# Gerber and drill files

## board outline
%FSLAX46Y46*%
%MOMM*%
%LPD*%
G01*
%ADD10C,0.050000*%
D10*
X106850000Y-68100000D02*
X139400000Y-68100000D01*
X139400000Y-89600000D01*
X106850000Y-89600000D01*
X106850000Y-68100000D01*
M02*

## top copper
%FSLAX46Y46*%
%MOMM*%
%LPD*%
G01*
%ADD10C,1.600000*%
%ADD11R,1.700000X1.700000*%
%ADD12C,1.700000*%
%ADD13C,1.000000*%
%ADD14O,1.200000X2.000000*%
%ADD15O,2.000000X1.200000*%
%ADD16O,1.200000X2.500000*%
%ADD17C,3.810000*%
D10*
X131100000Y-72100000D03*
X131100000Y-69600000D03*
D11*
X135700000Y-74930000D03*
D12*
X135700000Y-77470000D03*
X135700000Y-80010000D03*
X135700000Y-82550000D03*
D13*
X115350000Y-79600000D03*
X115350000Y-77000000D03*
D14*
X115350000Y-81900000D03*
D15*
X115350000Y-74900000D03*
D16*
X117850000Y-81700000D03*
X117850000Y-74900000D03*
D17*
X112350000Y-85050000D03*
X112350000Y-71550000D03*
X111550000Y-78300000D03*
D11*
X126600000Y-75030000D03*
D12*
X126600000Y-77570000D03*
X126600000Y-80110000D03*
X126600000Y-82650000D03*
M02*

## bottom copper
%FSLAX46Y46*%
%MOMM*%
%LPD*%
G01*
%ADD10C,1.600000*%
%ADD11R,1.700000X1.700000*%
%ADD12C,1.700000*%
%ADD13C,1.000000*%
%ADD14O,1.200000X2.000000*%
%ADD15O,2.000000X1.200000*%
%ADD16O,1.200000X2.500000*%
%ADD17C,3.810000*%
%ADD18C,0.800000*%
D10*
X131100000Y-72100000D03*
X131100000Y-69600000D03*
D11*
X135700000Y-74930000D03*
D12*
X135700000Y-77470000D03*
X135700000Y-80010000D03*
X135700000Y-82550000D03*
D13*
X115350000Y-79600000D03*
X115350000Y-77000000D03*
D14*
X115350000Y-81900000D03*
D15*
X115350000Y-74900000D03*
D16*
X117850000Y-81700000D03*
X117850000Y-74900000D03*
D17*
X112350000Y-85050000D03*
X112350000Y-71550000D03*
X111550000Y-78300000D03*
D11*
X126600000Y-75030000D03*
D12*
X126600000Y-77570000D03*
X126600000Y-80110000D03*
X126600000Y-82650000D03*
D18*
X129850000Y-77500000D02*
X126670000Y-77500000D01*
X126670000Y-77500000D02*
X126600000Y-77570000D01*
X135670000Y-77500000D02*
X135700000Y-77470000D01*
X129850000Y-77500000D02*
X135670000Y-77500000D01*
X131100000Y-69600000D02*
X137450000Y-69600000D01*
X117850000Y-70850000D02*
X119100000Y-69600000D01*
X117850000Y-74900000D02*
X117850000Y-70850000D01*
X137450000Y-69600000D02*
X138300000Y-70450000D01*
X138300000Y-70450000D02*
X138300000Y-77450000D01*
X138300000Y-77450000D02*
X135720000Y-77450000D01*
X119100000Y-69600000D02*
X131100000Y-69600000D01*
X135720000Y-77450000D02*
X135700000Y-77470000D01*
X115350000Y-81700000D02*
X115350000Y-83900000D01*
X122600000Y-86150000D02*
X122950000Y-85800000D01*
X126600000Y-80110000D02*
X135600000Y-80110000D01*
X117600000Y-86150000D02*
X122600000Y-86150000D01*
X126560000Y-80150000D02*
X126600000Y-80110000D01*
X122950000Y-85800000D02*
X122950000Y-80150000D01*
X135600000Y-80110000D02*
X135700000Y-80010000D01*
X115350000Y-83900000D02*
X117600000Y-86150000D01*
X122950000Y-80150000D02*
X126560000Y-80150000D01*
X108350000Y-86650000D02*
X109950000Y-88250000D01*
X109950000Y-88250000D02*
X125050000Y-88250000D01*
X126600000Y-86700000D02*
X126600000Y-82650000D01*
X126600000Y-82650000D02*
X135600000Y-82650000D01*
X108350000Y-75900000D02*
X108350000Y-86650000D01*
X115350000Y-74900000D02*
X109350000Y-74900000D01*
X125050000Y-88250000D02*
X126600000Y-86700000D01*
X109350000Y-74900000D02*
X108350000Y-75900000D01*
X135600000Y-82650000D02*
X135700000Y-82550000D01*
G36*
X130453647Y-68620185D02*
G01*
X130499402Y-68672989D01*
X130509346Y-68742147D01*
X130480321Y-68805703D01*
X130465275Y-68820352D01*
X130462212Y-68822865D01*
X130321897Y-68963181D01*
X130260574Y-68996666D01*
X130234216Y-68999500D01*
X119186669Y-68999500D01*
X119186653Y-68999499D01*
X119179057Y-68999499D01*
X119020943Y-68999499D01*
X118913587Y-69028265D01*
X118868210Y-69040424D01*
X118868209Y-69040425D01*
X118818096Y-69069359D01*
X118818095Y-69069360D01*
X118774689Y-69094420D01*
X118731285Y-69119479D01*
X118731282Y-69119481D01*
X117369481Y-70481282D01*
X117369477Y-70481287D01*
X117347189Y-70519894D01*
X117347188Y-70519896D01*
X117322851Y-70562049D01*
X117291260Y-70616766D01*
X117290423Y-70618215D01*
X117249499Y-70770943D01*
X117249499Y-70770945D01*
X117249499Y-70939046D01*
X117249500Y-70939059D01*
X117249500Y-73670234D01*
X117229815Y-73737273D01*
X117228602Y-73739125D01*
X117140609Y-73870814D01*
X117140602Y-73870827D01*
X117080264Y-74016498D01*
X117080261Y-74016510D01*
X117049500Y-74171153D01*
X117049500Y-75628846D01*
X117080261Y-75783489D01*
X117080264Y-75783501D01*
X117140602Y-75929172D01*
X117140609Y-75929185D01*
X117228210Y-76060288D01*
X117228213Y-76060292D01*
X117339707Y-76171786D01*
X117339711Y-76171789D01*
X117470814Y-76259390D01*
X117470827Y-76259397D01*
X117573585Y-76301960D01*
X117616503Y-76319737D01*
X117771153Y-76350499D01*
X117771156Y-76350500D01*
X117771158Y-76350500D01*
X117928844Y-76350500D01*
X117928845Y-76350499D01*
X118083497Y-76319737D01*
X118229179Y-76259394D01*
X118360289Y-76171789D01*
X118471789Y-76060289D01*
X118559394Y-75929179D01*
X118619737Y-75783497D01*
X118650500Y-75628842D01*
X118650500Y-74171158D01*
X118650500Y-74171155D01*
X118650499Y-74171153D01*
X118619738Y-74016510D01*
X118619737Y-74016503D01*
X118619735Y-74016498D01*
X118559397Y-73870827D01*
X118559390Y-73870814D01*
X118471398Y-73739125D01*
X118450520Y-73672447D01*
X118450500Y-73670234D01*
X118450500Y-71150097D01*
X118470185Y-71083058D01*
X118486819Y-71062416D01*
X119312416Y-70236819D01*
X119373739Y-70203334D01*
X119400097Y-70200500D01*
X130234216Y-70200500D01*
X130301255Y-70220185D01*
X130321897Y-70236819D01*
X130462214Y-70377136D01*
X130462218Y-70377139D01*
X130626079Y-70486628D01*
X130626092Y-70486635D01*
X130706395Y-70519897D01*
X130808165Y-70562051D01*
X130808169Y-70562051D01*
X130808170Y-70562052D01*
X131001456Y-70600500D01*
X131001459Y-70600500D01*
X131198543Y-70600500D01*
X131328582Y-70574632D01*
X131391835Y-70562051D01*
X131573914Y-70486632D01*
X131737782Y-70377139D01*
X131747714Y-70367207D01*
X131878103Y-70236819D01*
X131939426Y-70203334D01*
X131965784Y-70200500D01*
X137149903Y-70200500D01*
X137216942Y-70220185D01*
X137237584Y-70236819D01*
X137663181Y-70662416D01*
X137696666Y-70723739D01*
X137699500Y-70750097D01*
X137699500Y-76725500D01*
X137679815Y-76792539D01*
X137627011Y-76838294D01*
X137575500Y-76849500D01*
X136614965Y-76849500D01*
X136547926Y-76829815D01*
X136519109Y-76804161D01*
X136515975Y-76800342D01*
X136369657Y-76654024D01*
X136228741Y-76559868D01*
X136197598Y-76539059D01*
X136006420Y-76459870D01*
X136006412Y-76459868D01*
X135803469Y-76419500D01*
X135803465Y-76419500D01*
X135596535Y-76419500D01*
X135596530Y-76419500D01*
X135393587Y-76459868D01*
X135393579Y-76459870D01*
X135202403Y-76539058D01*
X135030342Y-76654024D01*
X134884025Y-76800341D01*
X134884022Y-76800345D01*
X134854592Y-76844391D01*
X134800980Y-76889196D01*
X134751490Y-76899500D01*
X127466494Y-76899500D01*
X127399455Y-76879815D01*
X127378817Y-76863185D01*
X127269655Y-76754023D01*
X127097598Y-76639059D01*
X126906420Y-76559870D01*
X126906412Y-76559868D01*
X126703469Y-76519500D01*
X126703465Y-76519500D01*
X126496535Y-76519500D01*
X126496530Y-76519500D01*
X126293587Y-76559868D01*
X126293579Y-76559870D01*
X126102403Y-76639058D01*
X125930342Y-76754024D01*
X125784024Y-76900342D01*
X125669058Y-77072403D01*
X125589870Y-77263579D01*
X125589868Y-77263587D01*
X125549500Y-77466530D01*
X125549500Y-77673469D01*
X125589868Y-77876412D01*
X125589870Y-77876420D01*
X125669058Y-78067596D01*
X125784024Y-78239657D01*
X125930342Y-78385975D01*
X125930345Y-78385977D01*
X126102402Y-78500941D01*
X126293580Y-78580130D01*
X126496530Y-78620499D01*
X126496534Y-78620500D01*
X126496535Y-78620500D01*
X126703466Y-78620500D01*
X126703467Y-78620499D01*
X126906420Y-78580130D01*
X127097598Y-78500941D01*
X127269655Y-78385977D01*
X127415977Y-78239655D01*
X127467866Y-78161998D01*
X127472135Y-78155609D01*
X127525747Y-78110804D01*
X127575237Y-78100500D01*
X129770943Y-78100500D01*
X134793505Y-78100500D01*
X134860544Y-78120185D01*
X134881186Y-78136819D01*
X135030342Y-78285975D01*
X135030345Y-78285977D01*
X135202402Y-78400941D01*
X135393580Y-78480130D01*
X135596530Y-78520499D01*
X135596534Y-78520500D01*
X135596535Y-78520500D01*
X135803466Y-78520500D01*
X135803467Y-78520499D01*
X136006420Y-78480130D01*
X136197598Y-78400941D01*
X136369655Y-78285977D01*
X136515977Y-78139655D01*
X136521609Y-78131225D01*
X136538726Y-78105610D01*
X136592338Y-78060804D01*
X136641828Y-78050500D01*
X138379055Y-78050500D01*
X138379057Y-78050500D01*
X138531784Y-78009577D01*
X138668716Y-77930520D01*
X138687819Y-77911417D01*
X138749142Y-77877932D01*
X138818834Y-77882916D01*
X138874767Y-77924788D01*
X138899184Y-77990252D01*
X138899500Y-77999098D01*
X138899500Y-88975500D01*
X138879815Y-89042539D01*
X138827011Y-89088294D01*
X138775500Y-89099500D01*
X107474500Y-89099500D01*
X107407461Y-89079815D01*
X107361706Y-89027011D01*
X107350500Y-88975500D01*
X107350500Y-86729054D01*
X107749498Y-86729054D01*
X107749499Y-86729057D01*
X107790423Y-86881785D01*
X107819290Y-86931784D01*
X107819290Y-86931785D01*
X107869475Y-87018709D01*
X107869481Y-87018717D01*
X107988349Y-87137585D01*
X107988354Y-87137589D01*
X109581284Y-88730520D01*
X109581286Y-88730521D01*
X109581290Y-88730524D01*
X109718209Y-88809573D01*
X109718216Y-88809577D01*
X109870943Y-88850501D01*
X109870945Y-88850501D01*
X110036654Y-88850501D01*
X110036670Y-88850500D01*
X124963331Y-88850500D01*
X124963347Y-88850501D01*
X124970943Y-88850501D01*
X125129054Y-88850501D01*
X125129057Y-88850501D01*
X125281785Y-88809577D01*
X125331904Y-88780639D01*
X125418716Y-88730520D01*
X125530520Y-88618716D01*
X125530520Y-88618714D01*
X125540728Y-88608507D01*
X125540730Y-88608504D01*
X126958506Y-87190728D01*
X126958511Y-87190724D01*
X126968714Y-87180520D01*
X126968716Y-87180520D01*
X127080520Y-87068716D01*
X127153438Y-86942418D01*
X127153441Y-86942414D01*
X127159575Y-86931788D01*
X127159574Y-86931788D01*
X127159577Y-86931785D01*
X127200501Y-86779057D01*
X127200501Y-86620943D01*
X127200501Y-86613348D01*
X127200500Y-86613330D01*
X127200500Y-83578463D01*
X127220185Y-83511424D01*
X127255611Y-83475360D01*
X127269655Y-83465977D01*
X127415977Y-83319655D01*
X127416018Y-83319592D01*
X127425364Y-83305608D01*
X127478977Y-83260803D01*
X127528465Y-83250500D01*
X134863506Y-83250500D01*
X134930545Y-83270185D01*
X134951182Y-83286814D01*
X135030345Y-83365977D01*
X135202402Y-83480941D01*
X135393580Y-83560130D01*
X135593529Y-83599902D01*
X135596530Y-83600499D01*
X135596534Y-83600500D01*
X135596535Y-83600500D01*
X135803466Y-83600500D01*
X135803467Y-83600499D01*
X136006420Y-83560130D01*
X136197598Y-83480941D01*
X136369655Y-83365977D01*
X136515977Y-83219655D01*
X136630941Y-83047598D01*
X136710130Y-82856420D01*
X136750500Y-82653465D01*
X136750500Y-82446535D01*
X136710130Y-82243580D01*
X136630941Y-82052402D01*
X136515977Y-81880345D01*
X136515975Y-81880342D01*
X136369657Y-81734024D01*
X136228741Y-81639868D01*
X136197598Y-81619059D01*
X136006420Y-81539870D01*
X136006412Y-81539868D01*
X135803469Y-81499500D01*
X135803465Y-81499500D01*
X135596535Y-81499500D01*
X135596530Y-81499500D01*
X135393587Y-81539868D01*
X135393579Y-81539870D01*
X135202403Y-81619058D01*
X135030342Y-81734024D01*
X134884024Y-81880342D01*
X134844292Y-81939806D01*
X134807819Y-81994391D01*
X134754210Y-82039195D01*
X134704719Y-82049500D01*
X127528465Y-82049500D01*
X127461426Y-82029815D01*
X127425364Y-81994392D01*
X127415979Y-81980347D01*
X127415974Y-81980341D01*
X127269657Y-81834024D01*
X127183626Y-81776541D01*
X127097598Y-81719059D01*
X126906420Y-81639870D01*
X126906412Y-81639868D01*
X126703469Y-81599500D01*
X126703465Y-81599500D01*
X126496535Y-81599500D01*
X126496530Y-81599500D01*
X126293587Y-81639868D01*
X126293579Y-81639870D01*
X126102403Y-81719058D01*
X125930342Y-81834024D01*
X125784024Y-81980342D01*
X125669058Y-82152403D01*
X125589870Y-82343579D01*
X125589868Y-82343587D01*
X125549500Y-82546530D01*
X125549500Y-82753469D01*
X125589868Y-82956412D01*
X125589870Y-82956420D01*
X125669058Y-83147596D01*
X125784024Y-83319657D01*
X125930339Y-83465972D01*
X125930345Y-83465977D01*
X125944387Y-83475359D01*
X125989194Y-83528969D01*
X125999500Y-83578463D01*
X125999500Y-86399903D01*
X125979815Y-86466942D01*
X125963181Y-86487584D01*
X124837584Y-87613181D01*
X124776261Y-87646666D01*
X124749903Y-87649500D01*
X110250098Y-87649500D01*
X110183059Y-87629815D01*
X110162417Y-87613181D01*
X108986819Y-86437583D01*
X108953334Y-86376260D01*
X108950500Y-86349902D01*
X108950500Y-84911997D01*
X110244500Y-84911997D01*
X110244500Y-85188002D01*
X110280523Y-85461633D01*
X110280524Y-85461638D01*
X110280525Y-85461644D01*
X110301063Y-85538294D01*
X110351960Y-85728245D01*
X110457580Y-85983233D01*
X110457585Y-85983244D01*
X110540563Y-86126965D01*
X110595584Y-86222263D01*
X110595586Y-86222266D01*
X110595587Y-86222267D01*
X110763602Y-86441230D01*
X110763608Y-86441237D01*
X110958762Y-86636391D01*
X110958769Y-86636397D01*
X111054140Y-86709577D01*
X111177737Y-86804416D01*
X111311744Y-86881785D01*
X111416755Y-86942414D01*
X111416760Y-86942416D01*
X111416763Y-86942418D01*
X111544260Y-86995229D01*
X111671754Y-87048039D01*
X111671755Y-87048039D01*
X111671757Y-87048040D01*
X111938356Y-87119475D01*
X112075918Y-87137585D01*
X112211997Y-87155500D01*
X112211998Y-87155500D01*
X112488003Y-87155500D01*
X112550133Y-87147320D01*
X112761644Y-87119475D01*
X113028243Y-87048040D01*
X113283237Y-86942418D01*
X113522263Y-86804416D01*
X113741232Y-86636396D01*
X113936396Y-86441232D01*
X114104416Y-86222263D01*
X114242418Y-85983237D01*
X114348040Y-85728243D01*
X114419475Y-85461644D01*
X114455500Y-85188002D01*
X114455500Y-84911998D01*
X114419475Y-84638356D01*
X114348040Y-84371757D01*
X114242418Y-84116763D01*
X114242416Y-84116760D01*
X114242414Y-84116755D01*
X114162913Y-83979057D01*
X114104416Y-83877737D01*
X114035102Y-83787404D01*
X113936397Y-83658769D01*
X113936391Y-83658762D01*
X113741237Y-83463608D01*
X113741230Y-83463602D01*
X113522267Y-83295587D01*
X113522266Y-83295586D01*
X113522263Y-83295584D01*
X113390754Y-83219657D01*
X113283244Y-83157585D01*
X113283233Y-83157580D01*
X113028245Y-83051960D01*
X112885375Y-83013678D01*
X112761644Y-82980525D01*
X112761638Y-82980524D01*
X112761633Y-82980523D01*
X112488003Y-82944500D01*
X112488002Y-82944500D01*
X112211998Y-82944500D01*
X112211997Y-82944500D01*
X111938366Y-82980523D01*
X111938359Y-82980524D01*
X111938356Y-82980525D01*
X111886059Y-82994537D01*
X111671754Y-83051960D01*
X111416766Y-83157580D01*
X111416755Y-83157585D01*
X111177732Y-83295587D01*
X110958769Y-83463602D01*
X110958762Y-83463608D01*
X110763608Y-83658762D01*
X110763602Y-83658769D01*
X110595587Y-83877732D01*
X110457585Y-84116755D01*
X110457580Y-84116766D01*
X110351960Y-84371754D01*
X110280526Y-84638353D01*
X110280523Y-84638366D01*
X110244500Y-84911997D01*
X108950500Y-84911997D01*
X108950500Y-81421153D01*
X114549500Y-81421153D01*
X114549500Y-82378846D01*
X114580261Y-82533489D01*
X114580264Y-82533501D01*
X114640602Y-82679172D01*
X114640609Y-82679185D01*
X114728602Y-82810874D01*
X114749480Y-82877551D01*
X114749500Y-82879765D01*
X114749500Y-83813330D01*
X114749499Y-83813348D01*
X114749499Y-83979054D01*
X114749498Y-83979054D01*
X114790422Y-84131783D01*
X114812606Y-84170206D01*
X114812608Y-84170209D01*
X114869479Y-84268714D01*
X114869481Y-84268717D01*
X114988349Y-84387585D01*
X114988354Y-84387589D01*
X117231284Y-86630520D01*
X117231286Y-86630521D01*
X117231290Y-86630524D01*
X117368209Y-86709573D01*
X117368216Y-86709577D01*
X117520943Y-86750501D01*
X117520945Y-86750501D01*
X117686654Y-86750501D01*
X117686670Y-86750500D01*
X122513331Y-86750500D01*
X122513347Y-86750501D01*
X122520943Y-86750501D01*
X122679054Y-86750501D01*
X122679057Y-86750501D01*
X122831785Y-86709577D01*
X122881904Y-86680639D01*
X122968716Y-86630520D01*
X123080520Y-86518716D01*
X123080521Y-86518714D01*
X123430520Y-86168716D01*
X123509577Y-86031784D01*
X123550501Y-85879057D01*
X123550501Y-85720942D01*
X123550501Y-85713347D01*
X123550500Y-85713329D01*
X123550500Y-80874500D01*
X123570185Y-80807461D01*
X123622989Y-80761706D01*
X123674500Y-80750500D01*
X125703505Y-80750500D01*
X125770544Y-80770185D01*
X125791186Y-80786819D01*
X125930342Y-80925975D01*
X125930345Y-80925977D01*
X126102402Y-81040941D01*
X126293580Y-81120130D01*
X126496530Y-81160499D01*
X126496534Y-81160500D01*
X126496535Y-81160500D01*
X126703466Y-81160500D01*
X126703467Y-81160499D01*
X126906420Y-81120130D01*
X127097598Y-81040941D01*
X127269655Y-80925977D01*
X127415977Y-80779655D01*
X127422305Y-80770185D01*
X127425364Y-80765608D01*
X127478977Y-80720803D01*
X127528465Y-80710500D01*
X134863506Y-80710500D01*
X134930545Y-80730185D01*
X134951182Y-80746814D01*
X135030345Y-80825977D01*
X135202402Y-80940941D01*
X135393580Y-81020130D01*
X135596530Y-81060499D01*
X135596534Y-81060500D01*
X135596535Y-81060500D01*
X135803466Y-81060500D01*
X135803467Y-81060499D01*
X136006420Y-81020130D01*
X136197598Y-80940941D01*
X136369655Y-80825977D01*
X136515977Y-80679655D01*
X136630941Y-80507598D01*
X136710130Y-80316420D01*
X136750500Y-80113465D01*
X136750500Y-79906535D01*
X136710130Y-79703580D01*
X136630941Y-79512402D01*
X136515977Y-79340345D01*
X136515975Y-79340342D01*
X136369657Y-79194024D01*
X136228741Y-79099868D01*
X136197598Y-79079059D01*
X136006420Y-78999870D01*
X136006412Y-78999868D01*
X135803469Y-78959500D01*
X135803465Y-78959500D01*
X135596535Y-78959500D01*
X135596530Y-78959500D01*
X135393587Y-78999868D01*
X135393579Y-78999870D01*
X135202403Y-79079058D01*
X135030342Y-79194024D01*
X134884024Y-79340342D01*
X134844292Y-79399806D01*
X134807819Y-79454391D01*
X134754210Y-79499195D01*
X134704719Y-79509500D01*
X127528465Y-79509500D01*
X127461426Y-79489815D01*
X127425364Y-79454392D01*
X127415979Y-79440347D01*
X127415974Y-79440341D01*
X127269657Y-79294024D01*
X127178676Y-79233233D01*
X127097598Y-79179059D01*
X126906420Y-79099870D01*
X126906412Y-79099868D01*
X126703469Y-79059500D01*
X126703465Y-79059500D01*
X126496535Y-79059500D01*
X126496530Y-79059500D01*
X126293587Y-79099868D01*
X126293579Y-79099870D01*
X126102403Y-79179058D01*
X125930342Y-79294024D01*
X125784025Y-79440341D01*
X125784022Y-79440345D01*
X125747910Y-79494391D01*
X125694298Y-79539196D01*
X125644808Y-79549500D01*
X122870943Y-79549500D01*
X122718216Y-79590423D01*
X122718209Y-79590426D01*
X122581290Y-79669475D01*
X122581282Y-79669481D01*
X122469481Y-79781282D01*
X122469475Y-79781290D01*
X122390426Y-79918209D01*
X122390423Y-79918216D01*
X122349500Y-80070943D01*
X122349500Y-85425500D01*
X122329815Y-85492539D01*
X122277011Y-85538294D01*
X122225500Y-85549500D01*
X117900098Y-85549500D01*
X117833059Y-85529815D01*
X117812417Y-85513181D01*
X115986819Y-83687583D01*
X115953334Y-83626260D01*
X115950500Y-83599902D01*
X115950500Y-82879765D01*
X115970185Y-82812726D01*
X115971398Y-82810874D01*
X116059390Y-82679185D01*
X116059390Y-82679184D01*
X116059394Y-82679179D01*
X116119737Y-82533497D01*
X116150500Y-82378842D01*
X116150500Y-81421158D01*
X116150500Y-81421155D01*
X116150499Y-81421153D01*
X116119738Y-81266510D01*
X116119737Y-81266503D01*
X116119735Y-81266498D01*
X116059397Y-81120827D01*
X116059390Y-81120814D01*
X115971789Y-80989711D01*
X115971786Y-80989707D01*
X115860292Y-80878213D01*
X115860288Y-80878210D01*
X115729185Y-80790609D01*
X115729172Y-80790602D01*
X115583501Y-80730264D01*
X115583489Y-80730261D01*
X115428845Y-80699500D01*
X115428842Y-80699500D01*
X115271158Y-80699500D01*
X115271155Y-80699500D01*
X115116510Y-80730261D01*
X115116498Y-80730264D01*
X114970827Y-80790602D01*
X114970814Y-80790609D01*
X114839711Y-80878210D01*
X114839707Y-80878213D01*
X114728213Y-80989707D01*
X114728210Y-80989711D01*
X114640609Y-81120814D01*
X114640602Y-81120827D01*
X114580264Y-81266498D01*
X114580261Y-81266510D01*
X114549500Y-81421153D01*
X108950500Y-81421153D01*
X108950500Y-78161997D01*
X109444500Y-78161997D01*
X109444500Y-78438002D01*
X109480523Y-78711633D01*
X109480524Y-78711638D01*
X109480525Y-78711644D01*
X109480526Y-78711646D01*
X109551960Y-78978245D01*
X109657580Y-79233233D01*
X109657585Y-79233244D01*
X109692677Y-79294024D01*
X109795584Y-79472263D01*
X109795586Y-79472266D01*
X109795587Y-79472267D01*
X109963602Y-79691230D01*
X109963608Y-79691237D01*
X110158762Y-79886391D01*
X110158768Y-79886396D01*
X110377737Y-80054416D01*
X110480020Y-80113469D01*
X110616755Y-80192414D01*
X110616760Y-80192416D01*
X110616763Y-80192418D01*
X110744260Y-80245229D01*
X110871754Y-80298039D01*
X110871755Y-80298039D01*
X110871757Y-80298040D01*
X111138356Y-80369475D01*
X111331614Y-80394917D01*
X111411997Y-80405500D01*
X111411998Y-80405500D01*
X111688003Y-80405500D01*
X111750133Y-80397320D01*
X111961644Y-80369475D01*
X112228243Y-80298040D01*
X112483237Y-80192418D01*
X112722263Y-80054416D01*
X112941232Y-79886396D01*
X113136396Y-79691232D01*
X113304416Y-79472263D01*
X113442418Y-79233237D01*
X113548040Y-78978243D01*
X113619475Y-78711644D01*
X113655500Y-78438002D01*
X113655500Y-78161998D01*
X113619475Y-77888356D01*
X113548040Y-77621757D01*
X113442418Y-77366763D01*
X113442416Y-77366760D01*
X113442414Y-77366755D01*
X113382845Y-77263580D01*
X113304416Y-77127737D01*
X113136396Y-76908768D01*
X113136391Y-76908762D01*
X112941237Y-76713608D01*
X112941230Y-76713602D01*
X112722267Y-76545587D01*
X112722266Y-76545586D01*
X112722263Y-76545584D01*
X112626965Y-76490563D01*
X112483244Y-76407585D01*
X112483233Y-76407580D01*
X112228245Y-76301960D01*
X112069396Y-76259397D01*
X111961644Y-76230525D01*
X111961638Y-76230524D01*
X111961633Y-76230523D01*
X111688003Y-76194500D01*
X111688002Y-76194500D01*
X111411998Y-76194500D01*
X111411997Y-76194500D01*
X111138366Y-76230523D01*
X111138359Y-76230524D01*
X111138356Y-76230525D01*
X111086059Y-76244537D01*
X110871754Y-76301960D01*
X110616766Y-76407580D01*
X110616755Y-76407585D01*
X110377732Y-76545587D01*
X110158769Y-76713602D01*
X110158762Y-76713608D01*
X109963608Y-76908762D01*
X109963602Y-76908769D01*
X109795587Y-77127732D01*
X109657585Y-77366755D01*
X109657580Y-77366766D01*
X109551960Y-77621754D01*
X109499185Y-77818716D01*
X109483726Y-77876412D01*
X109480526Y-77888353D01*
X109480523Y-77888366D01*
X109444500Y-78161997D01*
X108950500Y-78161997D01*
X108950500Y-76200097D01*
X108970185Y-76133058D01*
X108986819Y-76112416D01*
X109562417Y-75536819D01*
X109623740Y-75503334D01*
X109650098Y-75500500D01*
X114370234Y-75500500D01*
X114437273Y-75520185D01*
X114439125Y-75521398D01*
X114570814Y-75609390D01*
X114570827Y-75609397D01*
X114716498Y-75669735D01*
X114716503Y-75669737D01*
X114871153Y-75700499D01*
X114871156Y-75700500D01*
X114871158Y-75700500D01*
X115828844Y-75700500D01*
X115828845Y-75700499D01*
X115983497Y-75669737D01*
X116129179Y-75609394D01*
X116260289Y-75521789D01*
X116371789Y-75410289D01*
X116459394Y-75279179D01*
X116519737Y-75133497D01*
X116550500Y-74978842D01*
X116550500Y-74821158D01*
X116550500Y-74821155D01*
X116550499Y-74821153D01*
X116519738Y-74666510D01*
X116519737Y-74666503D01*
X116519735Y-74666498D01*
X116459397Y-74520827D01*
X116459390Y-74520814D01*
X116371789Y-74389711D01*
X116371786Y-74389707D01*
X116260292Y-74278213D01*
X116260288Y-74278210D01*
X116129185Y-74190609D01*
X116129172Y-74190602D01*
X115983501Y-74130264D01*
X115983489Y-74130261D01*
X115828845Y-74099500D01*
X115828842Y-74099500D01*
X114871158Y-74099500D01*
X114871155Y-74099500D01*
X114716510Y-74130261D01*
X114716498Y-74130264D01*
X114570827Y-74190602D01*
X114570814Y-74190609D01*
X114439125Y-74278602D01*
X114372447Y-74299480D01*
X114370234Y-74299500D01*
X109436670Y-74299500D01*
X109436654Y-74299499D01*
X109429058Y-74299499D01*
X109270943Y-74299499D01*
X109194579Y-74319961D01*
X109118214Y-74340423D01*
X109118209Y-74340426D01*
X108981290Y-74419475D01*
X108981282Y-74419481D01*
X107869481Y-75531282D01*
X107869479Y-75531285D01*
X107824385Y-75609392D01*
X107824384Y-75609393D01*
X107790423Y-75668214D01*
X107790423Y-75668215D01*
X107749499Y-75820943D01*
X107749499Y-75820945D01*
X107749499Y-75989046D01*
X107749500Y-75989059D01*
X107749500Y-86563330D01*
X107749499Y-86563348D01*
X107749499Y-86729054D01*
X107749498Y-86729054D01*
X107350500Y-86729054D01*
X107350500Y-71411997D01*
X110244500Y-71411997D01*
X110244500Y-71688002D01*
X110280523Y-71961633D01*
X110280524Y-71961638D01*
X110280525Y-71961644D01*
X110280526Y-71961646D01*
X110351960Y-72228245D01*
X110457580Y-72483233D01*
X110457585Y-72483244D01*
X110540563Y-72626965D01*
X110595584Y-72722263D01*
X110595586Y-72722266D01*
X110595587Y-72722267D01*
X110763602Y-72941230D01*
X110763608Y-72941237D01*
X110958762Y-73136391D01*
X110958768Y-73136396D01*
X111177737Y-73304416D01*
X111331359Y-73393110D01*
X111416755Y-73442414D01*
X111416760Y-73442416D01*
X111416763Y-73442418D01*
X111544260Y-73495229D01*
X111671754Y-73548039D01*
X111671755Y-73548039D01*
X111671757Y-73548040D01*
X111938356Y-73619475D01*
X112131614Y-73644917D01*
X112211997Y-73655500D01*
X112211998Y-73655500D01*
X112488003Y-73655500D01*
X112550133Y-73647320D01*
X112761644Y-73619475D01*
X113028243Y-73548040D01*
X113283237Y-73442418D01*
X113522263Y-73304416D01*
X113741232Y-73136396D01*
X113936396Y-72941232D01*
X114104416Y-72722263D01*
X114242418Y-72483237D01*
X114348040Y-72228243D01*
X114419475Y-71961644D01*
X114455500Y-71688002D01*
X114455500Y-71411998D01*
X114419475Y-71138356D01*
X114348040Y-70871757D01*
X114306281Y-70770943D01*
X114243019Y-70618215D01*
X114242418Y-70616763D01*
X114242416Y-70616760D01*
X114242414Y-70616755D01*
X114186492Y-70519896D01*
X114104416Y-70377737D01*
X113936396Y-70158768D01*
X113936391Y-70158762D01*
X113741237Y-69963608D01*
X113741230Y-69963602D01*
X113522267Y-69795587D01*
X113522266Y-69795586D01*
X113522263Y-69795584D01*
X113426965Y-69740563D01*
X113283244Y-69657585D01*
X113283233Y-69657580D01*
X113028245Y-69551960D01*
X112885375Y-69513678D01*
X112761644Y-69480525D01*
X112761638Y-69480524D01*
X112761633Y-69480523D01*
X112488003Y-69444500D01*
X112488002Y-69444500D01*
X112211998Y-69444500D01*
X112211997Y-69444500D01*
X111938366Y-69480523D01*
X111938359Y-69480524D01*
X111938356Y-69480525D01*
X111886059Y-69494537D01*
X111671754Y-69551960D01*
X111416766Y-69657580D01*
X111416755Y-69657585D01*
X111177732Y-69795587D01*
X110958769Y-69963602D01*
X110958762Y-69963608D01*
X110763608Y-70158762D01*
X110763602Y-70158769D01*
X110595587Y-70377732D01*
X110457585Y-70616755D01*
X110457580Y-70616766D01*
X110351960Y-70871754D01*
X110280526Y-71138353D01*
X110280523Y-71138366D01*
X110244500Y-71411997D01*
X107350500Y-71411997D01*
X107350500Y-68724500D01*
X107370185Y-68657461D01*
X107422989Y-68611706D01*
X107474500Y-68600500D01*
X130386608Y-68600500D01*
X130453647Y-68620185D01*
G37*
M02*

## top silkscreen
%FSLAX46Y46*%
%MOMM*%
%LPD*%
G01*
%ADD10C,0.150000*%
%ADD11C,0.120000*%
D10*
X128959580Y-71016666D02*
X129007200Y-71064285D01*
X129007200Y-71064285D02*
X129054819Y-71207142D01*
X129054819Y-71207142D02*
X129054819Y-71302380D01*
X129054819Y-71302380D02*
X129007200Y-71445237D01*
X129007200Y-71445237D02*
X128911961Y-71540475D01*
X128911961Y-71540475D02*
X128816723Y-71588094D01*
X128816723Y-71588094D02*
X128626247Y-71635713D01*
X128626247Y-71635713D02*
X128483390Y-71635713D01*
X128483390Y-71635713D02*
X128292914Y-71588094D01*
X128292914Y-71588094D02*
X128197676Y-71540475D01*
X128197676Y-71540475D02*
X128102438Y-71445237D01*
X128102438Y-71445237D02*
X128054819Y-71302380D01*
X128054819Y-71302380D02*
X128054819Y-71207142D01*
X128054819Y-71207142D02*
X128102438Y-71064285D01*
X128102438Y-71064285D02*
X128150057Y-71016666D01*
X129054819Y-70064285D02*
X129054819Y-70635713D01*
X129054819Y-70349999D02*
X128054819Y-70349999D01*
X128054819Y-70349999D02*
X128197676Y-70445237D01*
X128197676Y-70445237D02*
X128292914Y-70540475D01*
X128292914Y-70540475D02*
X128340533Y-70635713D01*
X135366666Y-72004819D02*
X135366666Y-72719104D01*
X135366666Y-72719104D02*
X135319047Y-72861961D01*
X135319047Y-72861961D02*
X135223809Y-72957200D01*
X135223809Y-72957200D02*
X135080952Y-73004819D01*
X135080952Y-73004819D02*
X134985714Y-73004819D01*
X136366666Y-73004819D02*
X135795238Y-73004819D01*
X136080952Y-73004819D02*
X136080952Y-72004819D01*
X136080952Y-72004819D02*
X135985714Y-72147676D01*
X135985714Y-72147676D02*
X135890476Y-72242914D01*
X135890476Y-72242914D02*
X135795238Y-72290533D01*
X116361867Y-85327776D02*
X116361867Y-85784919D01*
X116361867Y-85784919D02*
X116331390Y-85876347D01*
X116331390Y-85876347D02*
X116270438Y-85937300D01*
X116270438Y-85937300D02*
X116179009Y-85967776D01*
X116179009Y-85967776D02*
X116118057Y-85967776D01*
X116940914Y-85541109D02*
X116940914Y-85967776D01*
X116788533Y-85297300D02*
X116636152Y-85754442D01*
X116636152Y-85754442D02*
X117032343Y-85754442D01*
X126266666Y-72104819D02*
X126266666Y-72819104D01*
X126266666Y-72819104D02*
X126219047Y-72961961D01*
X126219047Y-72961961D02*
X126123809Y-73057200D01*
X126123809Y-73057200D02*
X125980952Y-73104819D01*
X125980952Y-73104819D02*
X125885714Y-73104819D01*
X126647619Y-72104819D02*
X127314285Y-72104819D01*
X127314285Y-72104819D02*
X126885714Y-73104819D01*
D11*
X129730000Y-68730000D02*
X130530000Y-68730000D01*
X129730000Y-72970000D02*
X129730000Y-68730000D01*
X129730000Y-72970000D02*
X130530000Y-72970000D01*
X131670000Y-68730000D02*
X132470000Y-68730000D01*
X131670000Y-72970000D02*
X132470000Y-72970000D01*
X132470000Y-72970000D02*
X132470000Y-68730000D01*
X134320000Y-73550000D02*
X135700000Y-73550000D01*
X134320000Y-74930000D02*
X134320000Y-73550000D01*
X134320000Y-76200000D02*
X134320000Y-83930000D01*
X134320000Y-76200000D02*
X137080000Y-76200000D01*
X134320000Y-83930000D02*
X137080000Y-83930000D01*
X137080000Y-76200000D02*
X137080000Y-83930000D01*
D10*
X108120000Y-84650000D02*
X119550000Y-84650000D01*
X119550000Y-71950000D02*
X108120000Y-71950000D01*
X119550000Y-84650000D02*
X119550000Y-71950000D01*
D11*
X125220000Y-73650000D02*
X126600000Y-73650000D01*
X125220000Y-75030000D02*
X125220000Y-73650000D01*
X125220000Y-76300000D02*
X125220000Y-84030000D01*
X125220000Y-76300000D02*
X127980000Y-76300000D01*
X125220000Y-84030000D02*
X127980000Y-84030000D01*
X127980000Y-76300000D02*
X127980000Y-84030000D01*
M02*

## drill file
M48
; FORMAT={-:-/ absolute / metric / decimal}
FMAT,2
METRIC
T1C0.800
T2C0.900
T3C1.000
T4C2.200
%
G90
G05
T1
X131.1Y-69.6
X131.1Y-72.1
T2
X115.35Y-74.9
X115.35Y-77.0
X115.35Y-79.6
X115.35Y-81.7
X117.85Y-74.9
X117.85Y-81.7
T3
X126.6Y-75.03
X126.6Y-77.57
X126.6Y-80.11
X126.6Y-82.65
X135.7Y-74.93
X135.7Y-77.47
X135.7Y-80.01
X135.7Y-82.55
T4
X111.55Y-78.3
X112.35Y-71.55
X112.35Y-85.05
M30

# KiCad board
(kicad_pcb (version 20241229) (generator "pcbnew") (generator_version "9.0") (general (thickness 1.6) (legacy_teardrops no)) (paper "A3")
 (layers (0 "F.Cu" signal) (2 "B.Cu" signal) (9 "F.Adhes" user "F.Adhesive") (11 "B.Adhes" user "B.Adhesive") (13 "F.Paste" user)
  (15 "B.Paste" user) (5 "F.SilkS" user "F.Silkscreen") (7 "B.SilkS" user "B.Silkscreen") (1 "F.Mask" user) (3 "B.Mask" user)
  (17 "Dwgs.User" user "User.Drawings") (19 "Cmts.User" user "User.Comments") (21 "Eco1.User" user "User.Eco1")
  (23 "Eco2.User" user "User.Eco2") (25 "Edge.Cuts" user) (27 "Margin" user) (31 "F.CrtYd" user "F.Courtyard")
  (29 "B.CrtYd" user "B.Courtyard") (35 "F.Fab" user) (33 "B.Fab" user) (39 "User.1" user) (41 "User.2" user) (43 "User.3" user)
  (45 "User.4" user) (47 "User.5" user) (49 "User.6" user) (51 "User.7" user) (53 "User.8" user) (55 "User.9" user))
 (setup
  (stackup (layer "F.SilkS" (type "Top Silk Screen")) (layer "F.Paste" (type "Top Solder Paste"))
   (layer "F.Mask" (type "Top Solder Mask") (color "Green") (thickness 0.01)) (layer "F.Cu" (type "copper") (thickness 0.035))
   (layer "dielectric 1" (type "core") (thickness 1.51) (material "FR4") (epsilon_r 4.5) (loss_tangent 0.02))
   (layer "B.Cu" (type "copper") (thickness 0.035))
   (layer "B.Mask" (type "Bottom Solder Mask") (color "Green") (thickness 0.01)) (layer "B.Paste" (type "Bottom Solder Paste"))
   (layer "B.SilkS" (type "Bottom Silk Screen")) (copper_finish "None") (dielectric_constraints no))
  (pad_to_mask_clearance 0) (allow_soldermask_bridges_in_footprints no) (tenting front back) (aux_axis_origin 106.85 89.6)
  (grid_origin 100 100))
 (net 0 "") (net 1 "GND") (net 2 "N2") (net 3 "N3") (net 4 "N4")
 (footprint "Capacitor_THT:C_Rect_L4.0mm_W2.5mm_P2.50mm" (layer "F.Cu") (at 131.1 72.1 90)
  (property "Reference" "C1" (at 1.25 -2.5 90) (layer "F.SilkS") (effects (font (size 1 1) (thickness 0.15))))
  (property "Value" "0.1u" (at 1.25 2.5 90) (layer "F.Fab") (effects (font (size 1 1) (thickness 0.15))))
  (fp_line (start 3.37 -1.37) (end 3.37 -0.57) (stroke (width 0.12) (type solid)) (layer "F.SilkS"))
  (fp_line (start -0.87 -1.37) (end 3.37 -1.37) (stroke (width 0.12) (type solid)) (layer "F.SilkS"))
  (fp_line (start -0.87 -1.37) (end -0.87 -0.57) (stroke (width 0.12) (type solid)) (layer "F.SilkS"))
  (fp_line (start 3.37 0.57) (end 3.37 1.37) (stroke (width 0.12) (type solid)) (layer "F.SilkS"))
  (fp_line (start -0.87 0.57) (end -0.87 1.37) (stroke (width 0.12) (type solid)) (layer "F.SilkS"))
  (fp_line (start -0.87 1.37) (end 3.37 1.37) (stroke (width 0.12) (type solid)) (layer "F.SilkS"))
  (pad "1" thru_hole circle (at 0 0 90) (size 1.6 1.6) (drill 0.8) (layers "*.Cu" "*.Mask") (remove_unused_layers no) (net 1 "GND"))
  (pad "2" thru_hole circle (at 2.5 0 90) (size 1.6 1.6) (drill 0.8) (layers "*.Cu" "*.Mask") (remove_unused_layers no) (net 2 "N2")))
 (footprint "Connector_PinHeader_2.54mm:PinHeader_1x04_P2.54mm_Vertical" (layer "F.Cu") (at 135.7 74.93)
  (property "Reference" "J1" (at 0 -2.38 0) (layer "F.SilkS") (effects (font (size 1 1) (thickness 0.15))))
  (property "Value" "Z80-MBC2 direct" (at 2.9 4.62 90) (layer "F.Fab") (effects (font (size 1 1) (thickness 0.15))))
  (fp_line (start -1.38 -1.38) (end 0 -1.38) (stroke (width 0.12) (type solid)) (layer "F.SilkS"))
  (fp_line (start -1.38 0) (end -1.38 -1.38) (stroke (width 0.12) (type solid)) (layer "F.SilkS"))
  (fp_line (start -1.38 1.27) (end -1.38 9) (stroke (width 0.12) (type solid)) (layer "F.SilkS"))
  (fp_line (start -1.38 1.27) (end 1.38 1.27) (stroke (width 0.12) (type solid)) (layer "F.SilkS"))
  (fp_line (start -1.38 9) (end 1.38 9) (stroke (width 0.12) (type solid)) (layer "F.SilkS"))
  (fp_line (start 1.38 1.27) (end 1.38 9) (stroke (width 0.12) (type solid)) (layer "F.SilkS"))
  (pad "1" thru_hole rect (at 0 0) (size 1.7 1.7) (drill 1) (layers "*.Cu" "*.Mask") (remove_unused_layers no) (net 1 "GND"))
  (pad "2" thru_hole circle (at 0 2.54) (size 1.7 1.7) (drill 1) (layers "*.Cu" "*.Mask") (remove_unused_layers no) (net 2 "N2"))
  (pad "3" thru_hole circle (at 0 5.08) (size 1.7 1.7) (drill 1) (layers "*.Cu" "*.Mask") (remove_unused_layers no) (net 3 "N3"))
  (pad "4" thru_hole circle (at 0 7.62) (size 1.7 1.7) (drill 1) (layers "*.Cu" "*.Mask") (remove_unused_layers no) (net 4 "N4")))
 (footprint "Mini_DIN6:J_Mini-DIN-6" (layer "F.Cu") (at 106.85 78.3 90)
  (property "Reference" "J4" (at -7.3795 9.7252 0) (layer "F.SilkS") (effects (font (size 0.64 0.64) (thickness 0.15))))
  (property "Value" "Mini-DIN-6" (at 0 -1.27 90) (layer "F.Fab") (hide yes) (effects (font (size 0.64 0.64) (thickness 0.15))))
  (fp_line (start -6.35 1.27) (end -6.35 12.7) (stroke (width 0.15) (type solid)) (layer "F.SilkS"))
  (fp_line (start 6.35 12.7) (end 6.35 1.27) (stroke (width 0.15) (type solid)) (layer "F.SilkS"))
  (fp_line (start -6.35 12.7) (end 6.35 12.7) (stroke (width 0.15) (type solid)) (layer "F.SilkS"))
  (pad "1" thru_hole circle (at -1.3 8.5 90) (size 1 1) (drill 0.9) (layers "*.Cu" "*.Mask") (remove_unused_layers no) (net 1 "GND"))
  (pad "2" thru_hole circle (at 1.3 8.5 90) (size 1 1) (drill 0.9) (layers "*.Cu" "*.Mask") (remove_unused_layers no) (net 1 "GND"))
  (pad "3" thru_hole oval (at -3.4 8.5 90) (size 2 1.2) (drill 0.9 (offset -0.2 0)) (layers "*.Cu" "*.Mask") (remove_unused_layers no)
   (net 3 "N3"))
  (pad "4" thru_hole oval (at 3.4 8.5 90) (size 1.2 2) (drill 0.9) (layers "*.Cu" "*.Mask") (remove_unused_layers no) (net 4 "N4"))
  (pad "5" thru_hole oval (at -3.4 11 90) (size 2.5 1.2) (drill 0.9) (layers "*.Cu" "*.Mask") (remove_unused_layers no) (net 1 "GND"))
  (pad "6" thru_hole oval (at 3.4 11 90) (size 2.5 1.2) (drill 0.9) (layers "*.Cu" "*.Mask") (remove_unused_layers no) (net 2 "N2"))
  (pad "C1" thru_hole circle (at -6.75 5.5 90) (size 3.81 3.81) (drill 2.2) (layers "*.Cu" "*.Mask") (remove_unused_layers no))
  (pad "C2" thru_hole circle (at 6.75 5.5 90) (size 3.81 3.81) (drill 2.2) (layers "*.Cu" "*.Mask") (remove_unused_layers no))
  (pad "SH" thru_hole circle (at 0 4.7 90) (size 3.81 3.81) (drill 2.2) (layers "*.Cu" "*.Mask") (remove_unused_layers no)))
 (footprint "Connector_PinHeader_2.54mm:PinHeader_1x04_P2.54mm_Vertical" (layer "F.Cu") (at 126.6 75.03)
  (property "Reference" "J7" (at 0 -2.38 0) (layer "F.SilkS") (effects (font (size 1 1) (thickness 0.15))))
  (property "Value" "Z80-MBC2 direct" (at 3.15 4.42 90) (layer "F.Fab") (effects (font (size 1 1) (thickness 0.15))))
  (fp_line (start -1.38 -1.38) (end 0 -1.38) (stroke (width 0.12) (type solid)) (layer "F.SilkS"))
  (fp_line (start -1.38 0) (end -1.38 -1.38) (stroke (width 0.12) (type solid)) (layer "F.SilkS"))
  (fp_line (start -1.38 1.27) (end -1.38 9) (stroke (width 0.12) (type solid)) (layer "F.SilkS"))
  (fp_line (start -1.38 1.27) (end 1.38 1.27) (stroke (width 0.12) (type solid)) (layer "F.SilkS"))
  (fp_line (start -1.38 9) (end 1.38 9) (stroke (width 0.12) (type solid)) (layer "F.SilkS"))
  (fp_line (start 1.38 1.27) (end 1.38 9) (stroke (width 0.12) (type solid)) (layer "F.SilkS"))
  (pad "1" thru_hole rect (at 0 0) (size 1.7 1.7) (drill 1) (layers "*.Cu" "*.Mask") (remove_unused_layers no) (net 1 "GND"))
  (pad "2" thru_hole circle (at 0 2.54) (size 1.7 1.7) (drill 1) (layers "*.Cu" "*.Mask") (remove_unused_layers no) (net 2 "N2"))
  (pad "3" thru_hole circle (at 0 5.08) (size 1.7 1.7) (drill 1) (layers "*.Cu" "*.Mask") (remove_unused_layers no) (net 3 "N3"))
  (pad "4" thru_hole circle (at 0 7.62) (size 1.7 1.7) (drill 1) (layers "*.Cu" "*.Mask") (remove_unused_layers no) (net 4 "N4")))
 (gr_rect (start 106.85 68.1) (end 139.4 89.6) (stroke (width 0.05) (type default)) (fill no) (layer "Edge.Cuts"))
 (segment (start 129.85 77.5) (end 126.67 77.5) (width 0.8) (layer "B.Cu") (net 2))
 (segment (start 126.67 77.5) (end 126.6 77.57) (width 0.8) (layer "B.Cu") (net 2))
 (segment (start 135.67 77.5) (end 135.7 77.47) (width 0.8) (layer "B.Cu") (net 2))
 (segment (start 129.85 77.5) (end 135.67 77.5) (width 0.8) (layer "B.Cu") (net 2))
 (segment (start 131.1 69.6) (end 137.45 69.6) (width 0.8) (layer "B.Cu") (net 2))
 (segment (start 117.85 70.85) (end 119.1 69.6) (width 0.8) (layer "B.Cu") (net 2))
 (segment (start 117.85 74.9) (end 117.85 70.85) (width 0.8) (layer "B.Cu") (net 2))
 (segment (start 137.45 69.6) (end 138.3 70.45) (width 0.8) (layer "B.Cu") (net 2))
 (segment (start 138.3 70.45) (end 138.3 77.45) (width 0.8) (layer "B.Cu") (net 2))
 (segment (start 138.3 77.45) (end 135.72 77.45) (width 0.8) (layer "B.Cu") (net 2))
 (segment (start 119.1 69.6) (end 131.1 69.6) (width 0.8) (layer "B.Cu") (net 2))
 (segment (start 135.72 77.45) (end 135.7 77.47) (width 0.8) (layer "B.Cu") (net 2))
 (segment (start 115.35 81.7) (end 115.35 83.9) (width 0.8) (layer "B.Cu") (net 3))
 (segment (start 122.6 86.15) (end 122.95 85.8) (width 0.8) (layer "B.Cu") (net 3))
 (segment (start 126.6 80.11) (end 135.6 80.11) (width 0.8) (layer "B.Cu") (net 3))
 (segment (start 117.6 86.15) (end 122.6 86.15) (width 0.8) (layer "B.Cu") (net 3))
 (segment (start 126.56 80.15) (end 126.6 80.11) (width 0.8) (layer "B.Cu") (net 3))
 (segment (start 122.95 85.8) (end 122.95 80.15) (width 0.8) (layer "B.Cu") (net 3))
 (segment (start 135.6 80.11) (end 135.7 80.01) (width 0.8) (layer "B.Cu") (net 3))
 (segment (start 115.35 83.9) (end 117.6 86.15) (width 0.8) (layer "B.Cu") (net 3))
 (segment (start 122.95 80.15) (end 126.56 80.15) (width 0.8) (layer "B.Cu") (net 3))
 (segment (start 108.35 86.65) (end 109.95 88.25) (width 0.8) (layer "B.Cu") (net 4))
 (segment (start 109.95 88.25) (end 125.05 88.25) (width 0.8) (layer "B.Cu") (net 4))
 (segment (start 126.6 86.7) (end 126.6 82.65) (width 0.8) (layer "B.Cu") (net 4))
 (segment (start 126.6 82.65) (end 135.6 82.65) (width 0.8) (layer "B.Cu") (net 4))
 (segment (start 108.35 75.9) (end 108.35 86.65) (width 0.8) (layer "B.Cu") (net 4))
 (segment (start 115.35 74.9) (end 109.35 74.9) (width 0.8) (layer "B.Cu") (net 4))
 (segment (start 125.05 88.25) (end 126.6 86.7) (width 0.8) (layer "B.Cu") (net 4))
 (segment (start 109.35 74.9) (end 108.35 75.9) (width 0.8) (layer "B.Cu") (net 4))
 (segment (start 135.6 82.65) (end 135.7 82.55) (width 0.8) (layer "B.Cu") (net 4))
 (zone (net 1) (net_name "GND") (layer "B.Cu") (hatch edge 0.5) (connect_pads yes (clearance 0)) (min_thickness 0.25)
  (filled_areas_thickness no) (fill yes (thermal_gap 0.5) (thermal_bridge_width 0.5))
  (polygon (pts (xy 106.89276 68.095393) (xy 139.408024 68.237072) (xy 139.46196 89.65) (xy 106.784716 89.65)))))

